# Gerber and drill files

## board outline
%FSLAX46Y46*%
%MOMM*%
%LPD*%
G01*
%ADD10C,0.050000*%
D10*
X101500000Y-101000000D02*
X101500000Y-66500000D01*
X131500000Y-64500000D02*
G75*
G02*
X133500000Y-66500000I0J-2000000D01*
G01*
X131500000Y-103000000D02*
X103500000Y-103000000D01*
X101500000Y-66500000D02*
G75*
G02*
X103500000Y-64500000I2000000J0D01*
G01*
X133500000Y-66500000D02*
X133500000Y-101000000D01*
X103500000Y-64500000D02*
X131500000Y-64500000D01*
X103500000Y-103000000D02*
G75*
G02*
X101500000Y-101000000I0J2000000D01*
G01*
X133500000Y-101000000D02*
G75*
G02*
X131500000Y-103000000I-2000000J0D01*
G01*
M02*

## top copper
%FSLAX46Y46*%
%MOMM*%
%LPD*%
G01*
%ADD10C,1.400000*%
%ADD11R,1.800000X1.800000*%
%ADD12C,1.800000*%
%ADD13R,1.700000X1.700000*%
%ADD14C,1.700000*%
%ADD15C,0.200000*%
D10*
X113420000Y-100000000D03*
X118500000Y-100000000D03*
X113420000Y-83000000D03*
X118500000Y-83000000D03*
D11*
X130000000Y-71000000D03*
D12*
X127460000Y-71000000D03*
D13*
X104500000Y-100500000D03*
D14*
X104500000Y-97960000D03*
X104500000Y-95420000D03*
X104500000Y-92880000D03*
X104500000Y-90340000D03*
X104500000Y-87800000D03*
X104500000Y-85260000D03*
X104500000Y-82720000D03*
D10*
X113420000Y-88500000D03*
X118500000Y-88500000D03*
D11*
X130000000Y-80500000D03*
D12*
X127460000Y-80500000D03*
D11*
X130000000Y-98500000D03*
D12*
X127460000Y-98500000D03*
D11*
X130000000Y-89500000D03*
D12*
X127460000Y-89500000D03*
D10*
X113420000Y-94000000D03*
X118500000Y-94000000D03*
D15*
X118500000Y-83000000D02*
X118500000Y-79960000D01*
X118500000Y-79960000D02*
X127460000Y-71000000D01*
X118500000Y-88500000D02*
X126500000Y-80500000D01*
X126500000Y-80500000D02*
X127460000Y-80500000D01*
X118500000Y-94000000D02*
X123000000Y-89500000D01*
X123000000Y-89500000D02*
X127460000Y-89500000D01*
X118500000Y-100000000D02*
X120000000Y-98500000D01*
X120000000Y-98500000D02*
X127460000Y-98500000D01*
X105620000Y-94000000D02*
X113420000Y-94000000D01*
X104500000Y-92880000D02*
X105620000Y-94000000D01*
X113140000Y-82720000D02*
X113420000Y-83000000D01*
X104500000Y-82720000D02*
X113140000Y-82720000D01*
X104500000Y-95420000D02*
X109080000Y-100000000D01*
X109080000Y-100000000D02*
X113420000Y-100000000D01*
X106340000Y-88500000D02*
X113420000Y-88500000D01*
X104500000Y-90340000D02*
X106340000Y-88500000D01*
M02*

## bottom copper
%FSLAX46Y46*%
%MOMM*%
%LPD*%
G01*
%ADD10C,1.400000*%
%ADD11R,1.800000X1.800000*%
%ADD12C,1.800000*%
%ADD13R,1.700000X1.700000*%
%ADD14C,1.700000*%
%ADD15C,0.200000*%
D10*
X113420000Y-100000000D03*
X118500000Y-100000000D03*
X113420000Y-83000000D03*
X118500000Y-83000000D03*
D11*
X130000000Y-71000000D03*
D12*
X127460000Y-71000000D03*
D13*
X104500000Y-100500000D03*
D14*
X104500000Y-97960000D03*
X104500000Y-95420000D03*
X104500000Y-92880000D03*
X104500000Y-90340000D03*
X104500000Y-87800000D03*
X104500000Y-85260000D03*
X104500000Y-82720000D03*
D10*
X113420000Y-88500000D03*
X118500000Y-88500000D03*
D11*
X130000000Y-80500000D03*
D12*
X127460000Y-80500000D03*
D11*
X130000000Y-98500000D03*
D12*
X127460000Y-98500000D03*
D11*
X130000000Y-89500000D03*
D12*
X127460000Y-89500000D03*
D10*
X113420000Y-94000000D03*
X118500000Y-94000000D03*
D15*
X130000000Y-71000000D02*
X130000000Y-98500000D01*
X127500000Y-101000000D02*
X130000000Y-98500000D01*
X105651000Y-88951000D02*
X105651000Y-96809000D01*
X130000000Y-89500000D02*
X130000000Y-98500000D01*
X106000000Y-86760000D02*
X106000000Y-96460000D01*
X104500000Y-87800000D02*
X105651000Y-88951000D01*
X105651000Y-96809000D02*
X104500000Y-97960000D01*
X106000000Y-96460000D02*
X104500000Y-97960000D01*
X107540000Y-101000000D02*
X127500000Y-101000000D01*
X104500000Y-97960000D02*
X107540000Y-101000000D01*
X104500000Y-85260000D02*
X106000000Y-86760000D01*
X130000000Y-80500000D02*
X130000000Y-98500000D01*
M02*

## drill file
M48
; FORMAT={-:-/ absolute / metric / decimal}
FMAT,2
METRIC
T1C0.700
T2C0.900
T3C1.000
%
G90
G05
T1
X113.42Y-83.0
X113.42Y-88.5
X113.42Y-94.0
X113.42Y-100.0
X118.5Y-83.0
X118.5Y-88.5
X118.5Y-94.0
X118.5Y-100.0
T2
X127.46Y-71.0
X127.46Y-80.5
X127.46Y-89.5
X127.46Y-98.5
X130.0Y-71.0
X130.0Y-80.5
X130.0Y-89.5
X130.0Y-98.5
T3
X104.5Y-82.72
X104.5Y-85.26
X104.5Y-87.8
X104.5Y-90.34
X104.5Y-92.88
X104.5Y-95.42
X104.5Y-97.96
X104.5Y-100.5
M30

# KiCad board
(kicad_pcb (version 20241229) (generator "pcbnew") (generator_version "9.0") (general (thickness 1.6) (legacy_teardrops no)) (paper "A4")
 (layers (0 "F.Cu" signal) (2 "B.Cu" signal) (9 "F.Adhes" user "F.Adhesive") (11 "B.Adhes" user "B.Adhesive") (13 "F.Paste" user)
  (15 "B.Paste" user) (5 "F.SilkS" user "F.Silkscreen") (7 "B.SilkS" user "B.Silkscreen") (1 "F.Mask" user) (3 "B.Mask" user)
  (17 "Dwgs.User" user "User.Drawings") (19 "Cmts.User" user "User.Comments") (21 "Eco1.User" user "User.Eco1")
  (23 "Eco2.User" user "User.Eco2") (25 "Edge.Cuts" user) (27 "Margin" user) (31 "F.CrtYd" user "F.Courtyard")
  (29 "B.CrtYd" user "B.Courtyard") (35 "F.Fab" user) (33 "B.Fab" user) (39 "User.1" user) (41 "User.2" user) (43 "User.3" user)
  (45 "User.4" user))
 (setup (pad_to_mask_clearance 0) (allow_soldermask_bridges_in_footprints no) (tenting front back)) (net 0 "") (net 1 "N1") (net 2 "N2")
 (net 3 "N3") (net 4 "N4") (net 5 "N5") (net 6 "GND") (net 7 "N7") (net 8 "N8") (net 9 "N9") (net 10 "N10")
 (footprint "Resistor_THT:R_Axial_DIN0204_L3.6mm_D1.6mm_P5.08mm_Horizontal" (layer "F.Cu") (at 113.42 100)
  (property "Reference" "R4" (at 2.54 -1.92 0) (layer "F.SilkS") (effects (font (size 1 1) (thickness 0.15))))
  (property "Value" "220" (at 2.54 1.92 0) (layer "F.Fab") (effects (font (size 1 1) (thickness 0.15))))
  (pad "1" thru_hole circle (at 0 0) (size 1.4 1.4) (drill 0.7) (layers "*.Cu" "*.Mask") (remove_unused_layers no) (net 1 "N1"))
  (pad "2" thru_hole circle (at 5.08 0) (size 1.4 1.4) (drill 0.7) (layers "*.Cu" "*.Mask") (remove_unused_layers no) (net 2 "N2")))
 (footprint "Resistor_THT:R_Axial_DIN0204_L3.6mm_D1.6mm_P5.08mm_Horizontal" (layer "F.Cu") (at 113.42 83)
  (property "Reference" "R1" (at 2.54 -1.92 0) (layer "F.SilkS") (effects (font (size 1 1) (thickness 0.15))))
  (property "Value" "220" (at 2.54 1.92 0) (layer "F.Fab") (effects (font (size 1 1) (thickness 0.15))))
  (pad "1" thru_hole circle (at 0 0) (size 1.4 1.4) (drill 0.7) (layers "*.Cu" "*.Mask") (remove_unused_layers no) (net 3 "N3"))
  (pad "2" thru_hole circle (at 5.08 0) (size 1.4 1.4) (drill 0.7) (layers "*.Cu" "*.Mask") (remove_unused_layers no) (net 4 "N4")))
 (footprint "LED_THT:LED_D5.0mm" (layer "F.Cu") (at 130 71 180)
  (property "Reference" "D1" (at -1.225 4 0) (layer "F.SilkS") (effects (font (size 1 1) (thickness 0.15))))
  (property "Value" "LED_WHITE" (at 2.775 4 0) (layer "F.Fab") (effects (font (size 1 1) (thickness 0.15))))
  (pad "1" thru_hole rect (at 0 0 180) (size 1.8 1.8) (drill 0.9) (layers "*.Cu" "*.Mask") (remove_unused_layers no) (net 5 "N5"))
  (pad "2" thru_hole circle (at 2.54 0 180) (size 1.8 1.8) (drill 0.9) (layers "*.Cu" "*.Mask") (remove_unused_layers no) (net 4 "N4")))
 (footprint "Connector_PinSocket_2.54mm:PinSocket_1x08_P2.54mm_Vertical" (layer "F.Cu") (at 104.5 100.5 180)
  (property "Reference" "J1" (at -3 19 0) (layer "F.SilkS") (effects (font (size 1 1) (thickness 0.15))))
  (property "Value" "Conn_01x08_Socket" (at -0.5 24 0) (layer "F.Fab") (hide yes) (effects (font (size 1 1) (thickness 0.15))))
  (pad "1" thru_hole rect (at 0 0 180) (size 1.7 1.7) (drill 1) (layers "*.Cu" "*.Mask") (remove_unused_layers no) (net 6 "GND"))
  (pad "2" thru_hole circle (at 0 2.54 180) (size 1.7 1.7) (drill 1) (layers "*.Cu" "*.Mask") (remove_unused_layers no) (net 5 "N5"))
  (pad "3" thru_hole circle (at 0 5.08 180) (size 1.7 1.7) (drill 1) (layers "*.Cu" "*.Mask") (remove_unused_layers no) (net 1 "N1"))
  (pad "4" thru_hole circle (at 0 7.62 180) (size 1.7 1.7) (drill 1) (layers "*.Cu" "*.Mask") (remove_unused_layers no) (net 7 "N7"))
  (pad "5" thru_hole circle (at 0 10.16 180) (size 1.7 1.7) (drill 1) (layers "*.Cu" "*.Mask") (remove_unused_layers no) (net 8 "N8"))
  (pad "6" thru_hole circle (at 0 12.7 180) (size 1.7 1.7) (drill 1) (layers "*.Cu" "*.Mask") (remove_unused_layers no) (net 5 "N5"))
  (pad "7" thru_hole circle (at 0 15.24 180) (size 1.7 1.7) (drill 1) (layers "*.Cu" "*.Mask") (remove_unused_layers no) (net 5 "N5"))
  (pad "8" thru_hole circle (at 0 17.78 180) (size 1.7 1.7) (drill 1) (layers "*.Cu" "*.Mask") (remove_unused_layers no) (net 3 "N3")))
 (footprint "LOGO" (layer "F.Cu") (at 119 70)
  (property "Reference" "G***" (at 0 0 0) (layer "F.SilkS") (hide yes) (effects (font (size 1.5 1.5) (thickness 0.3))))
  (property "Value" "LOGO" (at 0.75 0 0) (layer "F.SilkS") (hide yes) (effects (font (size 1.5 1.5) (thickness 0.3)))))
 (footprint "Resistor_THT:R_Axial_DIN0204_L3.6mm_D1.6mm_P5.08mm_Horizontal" (layer "F.Cu") (at 113.42 88.5)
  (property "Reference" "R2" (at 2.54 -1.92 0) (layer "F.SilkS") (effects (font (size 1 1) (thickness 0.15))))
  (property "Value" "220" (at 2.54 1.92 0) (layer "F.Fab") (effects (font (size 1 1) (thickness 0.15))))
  (pad "1" thru_hole circle (at 0 0) (size 1.4 1.4) (drill 0.7) (layers "*.Cu" "*.Mask") (remove_unused_layers no) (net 8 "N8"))
  (pad "2" thru_hole circle (at 5.08 0) (size 1.4 1.4) (drill 0.7) (layers "*.Cu" "*.Mask") (remove_unused_layers no) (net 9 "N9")))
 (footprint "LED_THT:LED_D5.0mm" (layer "F.Cu") (at 130 80.5 180)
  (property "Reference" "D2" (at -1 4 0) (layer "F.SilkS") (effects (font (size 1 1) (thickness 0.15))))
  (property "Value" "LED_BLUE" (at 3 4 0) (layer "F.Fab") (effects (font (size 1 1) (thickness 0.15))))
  (pad "1" thru_hole rect (at 0 0 180) (size 1.8 1.8) (drill 0.9) (layers "*.Cu" "*.Mask") (remove_unused_layers no) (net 5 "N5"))
  (pad "2" thru_hole circle (at 2.54 0 180) (size 1.8 1.8) (drill 0.9) (layers "*.Cu" "*.Mask") (remove_unused_layers no) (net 9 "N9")))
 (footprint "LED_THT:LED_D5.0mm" (layer "F.Cu") (at 130 98.5 180)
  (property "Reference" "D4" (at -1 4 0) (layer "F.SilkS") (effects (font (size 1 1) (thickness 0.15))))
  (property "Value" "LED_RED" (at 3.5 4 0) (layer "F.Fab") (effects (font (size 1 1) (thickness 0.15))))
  (pad "1" thru_hole rect (at 0 0 180) (size 1.8 1.8) (drill 0.9) (layers "*.Cu" "*.Mask") (remove_unused_layers no) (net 5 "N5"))
  (pad "2" thru_hole circle (at 2.54 0 180) (size 1.8 1.8) (drill 0.9) (layers "*.Cu" "*.Mask") (remove_unused_layers no) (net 2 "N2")))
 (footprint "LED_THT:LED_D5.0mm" (layer "F.Cu") (at 130 89.5 180)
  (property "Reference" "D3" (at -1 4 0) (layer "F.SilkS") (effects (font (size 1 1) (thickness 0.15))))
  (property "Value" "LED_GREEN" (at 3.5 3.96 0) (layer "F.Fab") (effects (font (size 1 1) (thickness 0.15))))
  (pad "1" thru_hole rect (at 0 0 180) (size 1.8 1.8) (drill 0.9) (layers "*.Cu" "*.Mask") (remove_unused_layers no) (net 5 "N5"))
  (pad "2" thru_hole circle (at 2.54 0 180) (size 1.8 1.8) (drill 0.9) (layers "*.Cu" "*.Mask") (remove_unused_layers no) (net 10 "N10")))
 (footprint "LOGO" (layer "F.Cu") (at 108 72)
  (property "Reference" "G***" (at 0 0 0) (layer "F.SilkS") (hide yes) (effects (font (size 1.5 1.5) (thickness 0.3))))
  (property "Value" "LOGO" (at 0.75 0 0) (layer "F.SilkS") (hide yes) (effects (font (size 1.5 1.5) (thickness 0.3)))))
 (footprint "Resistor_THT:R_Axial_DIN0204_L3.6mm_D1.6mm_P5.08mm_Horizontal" (layer "F.Cu") (at 113.42 94)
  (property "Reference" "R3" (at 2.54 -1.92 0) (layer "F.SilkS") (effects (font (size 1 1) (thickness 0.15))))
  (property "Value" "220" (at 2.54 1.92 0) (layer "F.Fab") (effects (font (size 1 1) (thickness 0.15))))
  (pad "1" thru_hole circle (at 0 0) (size 1.4 1.4) (drill 0.7) (layers "*.Cu" "*.Mask") (remove_unused_layers no) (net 7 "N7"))
  (pad "2" thru_hole circle (at 5.08 0) (size 1.4 1.4) (drill 0.7) (layers "*.Cu" "*.Mask") (remove_unused_layers no) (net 10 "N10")))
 (gr_line (start 101.5 101) (end 101.5 66.5) (stroke (width 0.05) (type default)) (layer "Edge.Cuts"))
 (gr_arc (start 131.5 64.5) (mid 132.914214 65.085786) (end 133.5 66.5) (stroke (width 0.05) (type default)) (layer "Edge.Cuts"))
 (gr_line (start 131.5 103) (end 103.5 103) (stroke (width 0.05) (type default)) (layer "Edge.Cuts"))
 (gr_arc (start 101.5 66.5) (mid 102.085786 65.085786) (end 103.5 64.5) (stroke (width 0.05) (type default)) (layer "Edge.Cuts"))
 (gr_line (start 133.5 66.5) (end 133.5 101) (stroke (width 0.05) (type default)) (layer "Edge.Cuts"))
 (gr_line (start 103.5 64.5) (end 131.5 64.5) (stroke (width 0.05) (type default)) (layer "Edge.Cuts"))
 (gr_arc (start 103.5 103) (mid 102.085786 102.414214) (end 101.5 101) (stroke (width 0.05) (type default)) (layer "Edge.Cuts"))
 (gr_arc (start 133.5 101) (mid 132.914214 102.414214) (end 131.5 103) (stroke (width 0.05) (type default)) (layer "Edge.Cuts"))
 (segment (start 130 71) (end 130 98.5) (width 0.2) (layer "B.Cu") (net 5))
 (segment (start 127.5 101) (end 130 98.5) (width 0.2) (layer "B.Cu") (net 5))
 (segment (start 105.651 88.951) (end 105.651 96.809) (width 0.2) (layer "B.Cu") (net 5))
 (segment (start 130 89.5) (end 130 98.5) (width 0.2) (layer "B.Cu") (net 5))
 (segment (start 106 86.76) (end 106 96.46) (width 0.2) (layer "B.Cu") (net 5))
 (segment (start 104.5 87.8) (end 105.651 88.951) (width 0.2) (layer "B.Cu") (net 5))
 (segment (start 105.651 96.809) (end 104.5 97.96) (width 0.2) (layer "B.Cu") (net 5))
 (segment (start 106 96.46) (end 104.5 97.96) (width 0.2) (layer "B.Cu") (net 5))
 (segment (start 107.54 101) (end 127.5 101) (width 0.2) (layer "B.Cu") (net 5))
 (segment (start 104.5 97.96) (end 107.54 101) (width 0.2) (layer "B.Cu") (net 5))
 (segment (start 104.5 85.26) (end 106 86.76) (width 0.2) (layer "B.Cu") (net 5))
 (segment (start 130 80.5) (end 130 98.5) (width 0.2) (layer "B.Cu") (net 5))
 (segment (start 118.5 83) (end 118.5 79.96) (width 0.2) (layer "F.Cu") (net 4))
 (segment (start 118.5 79.96) (end 127.46 71) (width 0.2) (layer "F.Cu") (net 4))
 (segment (start 118.5 88.5) (end 126.5 80.5) (width 0.2) (layer "F.Cu") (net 9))
 (segment (start 126.5 80.5) (end 127.46 80.5) (width 0.2) (layer "F.Cu") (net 9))
 (segment (start 118.5 94) (end 123 89.5) (width 0.2) (layer "F.Cu") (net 10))
 (segment (start 123 89.5) (end 127.46 89.5) (width 0.2) (layer "F.Cu") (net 10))
 (segment (start 118.5 100) (end 120 98.5) (width 0.2) (layer "F.Cu") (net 2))
 (segment (start 120 98.5) (end 127.46 98.5) (width 0.2) (layer "F.Cu") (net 2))
 (segment (start 105.62 94) (end 113.42 94) (width 0.2) (layer "F.Cu") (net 7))
 (segment (start 104.5 92.88) (end 105.62 94) (width 0.2) (layer "F.Cu") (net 7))
 (segment (start 113.14 82.72) (end 113.42 83) (width 0.2) (layer "F.Cu") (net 3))
 (segment (start 104.5 82.72) (end 113.14 82.72) (width 0.2) (layer "F.Cu") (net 3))
 (segment (start 104.5 95.42) (end 109.08 100) (width 0.2) (layer "F.Cu") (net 1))
 (segment (start 109.08 100) (end 113.42 100) (width 0.2) (layer "F.Cu") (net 1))
 (segment (start 106.34 88.5) (end 113.42 88.5) (width 0.2) (layer "F.Cu") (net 8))
 (segment (start 104.5 90.34) (end 106.34 88.5) (width 0.2) (layer "F.Cu") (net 8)))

